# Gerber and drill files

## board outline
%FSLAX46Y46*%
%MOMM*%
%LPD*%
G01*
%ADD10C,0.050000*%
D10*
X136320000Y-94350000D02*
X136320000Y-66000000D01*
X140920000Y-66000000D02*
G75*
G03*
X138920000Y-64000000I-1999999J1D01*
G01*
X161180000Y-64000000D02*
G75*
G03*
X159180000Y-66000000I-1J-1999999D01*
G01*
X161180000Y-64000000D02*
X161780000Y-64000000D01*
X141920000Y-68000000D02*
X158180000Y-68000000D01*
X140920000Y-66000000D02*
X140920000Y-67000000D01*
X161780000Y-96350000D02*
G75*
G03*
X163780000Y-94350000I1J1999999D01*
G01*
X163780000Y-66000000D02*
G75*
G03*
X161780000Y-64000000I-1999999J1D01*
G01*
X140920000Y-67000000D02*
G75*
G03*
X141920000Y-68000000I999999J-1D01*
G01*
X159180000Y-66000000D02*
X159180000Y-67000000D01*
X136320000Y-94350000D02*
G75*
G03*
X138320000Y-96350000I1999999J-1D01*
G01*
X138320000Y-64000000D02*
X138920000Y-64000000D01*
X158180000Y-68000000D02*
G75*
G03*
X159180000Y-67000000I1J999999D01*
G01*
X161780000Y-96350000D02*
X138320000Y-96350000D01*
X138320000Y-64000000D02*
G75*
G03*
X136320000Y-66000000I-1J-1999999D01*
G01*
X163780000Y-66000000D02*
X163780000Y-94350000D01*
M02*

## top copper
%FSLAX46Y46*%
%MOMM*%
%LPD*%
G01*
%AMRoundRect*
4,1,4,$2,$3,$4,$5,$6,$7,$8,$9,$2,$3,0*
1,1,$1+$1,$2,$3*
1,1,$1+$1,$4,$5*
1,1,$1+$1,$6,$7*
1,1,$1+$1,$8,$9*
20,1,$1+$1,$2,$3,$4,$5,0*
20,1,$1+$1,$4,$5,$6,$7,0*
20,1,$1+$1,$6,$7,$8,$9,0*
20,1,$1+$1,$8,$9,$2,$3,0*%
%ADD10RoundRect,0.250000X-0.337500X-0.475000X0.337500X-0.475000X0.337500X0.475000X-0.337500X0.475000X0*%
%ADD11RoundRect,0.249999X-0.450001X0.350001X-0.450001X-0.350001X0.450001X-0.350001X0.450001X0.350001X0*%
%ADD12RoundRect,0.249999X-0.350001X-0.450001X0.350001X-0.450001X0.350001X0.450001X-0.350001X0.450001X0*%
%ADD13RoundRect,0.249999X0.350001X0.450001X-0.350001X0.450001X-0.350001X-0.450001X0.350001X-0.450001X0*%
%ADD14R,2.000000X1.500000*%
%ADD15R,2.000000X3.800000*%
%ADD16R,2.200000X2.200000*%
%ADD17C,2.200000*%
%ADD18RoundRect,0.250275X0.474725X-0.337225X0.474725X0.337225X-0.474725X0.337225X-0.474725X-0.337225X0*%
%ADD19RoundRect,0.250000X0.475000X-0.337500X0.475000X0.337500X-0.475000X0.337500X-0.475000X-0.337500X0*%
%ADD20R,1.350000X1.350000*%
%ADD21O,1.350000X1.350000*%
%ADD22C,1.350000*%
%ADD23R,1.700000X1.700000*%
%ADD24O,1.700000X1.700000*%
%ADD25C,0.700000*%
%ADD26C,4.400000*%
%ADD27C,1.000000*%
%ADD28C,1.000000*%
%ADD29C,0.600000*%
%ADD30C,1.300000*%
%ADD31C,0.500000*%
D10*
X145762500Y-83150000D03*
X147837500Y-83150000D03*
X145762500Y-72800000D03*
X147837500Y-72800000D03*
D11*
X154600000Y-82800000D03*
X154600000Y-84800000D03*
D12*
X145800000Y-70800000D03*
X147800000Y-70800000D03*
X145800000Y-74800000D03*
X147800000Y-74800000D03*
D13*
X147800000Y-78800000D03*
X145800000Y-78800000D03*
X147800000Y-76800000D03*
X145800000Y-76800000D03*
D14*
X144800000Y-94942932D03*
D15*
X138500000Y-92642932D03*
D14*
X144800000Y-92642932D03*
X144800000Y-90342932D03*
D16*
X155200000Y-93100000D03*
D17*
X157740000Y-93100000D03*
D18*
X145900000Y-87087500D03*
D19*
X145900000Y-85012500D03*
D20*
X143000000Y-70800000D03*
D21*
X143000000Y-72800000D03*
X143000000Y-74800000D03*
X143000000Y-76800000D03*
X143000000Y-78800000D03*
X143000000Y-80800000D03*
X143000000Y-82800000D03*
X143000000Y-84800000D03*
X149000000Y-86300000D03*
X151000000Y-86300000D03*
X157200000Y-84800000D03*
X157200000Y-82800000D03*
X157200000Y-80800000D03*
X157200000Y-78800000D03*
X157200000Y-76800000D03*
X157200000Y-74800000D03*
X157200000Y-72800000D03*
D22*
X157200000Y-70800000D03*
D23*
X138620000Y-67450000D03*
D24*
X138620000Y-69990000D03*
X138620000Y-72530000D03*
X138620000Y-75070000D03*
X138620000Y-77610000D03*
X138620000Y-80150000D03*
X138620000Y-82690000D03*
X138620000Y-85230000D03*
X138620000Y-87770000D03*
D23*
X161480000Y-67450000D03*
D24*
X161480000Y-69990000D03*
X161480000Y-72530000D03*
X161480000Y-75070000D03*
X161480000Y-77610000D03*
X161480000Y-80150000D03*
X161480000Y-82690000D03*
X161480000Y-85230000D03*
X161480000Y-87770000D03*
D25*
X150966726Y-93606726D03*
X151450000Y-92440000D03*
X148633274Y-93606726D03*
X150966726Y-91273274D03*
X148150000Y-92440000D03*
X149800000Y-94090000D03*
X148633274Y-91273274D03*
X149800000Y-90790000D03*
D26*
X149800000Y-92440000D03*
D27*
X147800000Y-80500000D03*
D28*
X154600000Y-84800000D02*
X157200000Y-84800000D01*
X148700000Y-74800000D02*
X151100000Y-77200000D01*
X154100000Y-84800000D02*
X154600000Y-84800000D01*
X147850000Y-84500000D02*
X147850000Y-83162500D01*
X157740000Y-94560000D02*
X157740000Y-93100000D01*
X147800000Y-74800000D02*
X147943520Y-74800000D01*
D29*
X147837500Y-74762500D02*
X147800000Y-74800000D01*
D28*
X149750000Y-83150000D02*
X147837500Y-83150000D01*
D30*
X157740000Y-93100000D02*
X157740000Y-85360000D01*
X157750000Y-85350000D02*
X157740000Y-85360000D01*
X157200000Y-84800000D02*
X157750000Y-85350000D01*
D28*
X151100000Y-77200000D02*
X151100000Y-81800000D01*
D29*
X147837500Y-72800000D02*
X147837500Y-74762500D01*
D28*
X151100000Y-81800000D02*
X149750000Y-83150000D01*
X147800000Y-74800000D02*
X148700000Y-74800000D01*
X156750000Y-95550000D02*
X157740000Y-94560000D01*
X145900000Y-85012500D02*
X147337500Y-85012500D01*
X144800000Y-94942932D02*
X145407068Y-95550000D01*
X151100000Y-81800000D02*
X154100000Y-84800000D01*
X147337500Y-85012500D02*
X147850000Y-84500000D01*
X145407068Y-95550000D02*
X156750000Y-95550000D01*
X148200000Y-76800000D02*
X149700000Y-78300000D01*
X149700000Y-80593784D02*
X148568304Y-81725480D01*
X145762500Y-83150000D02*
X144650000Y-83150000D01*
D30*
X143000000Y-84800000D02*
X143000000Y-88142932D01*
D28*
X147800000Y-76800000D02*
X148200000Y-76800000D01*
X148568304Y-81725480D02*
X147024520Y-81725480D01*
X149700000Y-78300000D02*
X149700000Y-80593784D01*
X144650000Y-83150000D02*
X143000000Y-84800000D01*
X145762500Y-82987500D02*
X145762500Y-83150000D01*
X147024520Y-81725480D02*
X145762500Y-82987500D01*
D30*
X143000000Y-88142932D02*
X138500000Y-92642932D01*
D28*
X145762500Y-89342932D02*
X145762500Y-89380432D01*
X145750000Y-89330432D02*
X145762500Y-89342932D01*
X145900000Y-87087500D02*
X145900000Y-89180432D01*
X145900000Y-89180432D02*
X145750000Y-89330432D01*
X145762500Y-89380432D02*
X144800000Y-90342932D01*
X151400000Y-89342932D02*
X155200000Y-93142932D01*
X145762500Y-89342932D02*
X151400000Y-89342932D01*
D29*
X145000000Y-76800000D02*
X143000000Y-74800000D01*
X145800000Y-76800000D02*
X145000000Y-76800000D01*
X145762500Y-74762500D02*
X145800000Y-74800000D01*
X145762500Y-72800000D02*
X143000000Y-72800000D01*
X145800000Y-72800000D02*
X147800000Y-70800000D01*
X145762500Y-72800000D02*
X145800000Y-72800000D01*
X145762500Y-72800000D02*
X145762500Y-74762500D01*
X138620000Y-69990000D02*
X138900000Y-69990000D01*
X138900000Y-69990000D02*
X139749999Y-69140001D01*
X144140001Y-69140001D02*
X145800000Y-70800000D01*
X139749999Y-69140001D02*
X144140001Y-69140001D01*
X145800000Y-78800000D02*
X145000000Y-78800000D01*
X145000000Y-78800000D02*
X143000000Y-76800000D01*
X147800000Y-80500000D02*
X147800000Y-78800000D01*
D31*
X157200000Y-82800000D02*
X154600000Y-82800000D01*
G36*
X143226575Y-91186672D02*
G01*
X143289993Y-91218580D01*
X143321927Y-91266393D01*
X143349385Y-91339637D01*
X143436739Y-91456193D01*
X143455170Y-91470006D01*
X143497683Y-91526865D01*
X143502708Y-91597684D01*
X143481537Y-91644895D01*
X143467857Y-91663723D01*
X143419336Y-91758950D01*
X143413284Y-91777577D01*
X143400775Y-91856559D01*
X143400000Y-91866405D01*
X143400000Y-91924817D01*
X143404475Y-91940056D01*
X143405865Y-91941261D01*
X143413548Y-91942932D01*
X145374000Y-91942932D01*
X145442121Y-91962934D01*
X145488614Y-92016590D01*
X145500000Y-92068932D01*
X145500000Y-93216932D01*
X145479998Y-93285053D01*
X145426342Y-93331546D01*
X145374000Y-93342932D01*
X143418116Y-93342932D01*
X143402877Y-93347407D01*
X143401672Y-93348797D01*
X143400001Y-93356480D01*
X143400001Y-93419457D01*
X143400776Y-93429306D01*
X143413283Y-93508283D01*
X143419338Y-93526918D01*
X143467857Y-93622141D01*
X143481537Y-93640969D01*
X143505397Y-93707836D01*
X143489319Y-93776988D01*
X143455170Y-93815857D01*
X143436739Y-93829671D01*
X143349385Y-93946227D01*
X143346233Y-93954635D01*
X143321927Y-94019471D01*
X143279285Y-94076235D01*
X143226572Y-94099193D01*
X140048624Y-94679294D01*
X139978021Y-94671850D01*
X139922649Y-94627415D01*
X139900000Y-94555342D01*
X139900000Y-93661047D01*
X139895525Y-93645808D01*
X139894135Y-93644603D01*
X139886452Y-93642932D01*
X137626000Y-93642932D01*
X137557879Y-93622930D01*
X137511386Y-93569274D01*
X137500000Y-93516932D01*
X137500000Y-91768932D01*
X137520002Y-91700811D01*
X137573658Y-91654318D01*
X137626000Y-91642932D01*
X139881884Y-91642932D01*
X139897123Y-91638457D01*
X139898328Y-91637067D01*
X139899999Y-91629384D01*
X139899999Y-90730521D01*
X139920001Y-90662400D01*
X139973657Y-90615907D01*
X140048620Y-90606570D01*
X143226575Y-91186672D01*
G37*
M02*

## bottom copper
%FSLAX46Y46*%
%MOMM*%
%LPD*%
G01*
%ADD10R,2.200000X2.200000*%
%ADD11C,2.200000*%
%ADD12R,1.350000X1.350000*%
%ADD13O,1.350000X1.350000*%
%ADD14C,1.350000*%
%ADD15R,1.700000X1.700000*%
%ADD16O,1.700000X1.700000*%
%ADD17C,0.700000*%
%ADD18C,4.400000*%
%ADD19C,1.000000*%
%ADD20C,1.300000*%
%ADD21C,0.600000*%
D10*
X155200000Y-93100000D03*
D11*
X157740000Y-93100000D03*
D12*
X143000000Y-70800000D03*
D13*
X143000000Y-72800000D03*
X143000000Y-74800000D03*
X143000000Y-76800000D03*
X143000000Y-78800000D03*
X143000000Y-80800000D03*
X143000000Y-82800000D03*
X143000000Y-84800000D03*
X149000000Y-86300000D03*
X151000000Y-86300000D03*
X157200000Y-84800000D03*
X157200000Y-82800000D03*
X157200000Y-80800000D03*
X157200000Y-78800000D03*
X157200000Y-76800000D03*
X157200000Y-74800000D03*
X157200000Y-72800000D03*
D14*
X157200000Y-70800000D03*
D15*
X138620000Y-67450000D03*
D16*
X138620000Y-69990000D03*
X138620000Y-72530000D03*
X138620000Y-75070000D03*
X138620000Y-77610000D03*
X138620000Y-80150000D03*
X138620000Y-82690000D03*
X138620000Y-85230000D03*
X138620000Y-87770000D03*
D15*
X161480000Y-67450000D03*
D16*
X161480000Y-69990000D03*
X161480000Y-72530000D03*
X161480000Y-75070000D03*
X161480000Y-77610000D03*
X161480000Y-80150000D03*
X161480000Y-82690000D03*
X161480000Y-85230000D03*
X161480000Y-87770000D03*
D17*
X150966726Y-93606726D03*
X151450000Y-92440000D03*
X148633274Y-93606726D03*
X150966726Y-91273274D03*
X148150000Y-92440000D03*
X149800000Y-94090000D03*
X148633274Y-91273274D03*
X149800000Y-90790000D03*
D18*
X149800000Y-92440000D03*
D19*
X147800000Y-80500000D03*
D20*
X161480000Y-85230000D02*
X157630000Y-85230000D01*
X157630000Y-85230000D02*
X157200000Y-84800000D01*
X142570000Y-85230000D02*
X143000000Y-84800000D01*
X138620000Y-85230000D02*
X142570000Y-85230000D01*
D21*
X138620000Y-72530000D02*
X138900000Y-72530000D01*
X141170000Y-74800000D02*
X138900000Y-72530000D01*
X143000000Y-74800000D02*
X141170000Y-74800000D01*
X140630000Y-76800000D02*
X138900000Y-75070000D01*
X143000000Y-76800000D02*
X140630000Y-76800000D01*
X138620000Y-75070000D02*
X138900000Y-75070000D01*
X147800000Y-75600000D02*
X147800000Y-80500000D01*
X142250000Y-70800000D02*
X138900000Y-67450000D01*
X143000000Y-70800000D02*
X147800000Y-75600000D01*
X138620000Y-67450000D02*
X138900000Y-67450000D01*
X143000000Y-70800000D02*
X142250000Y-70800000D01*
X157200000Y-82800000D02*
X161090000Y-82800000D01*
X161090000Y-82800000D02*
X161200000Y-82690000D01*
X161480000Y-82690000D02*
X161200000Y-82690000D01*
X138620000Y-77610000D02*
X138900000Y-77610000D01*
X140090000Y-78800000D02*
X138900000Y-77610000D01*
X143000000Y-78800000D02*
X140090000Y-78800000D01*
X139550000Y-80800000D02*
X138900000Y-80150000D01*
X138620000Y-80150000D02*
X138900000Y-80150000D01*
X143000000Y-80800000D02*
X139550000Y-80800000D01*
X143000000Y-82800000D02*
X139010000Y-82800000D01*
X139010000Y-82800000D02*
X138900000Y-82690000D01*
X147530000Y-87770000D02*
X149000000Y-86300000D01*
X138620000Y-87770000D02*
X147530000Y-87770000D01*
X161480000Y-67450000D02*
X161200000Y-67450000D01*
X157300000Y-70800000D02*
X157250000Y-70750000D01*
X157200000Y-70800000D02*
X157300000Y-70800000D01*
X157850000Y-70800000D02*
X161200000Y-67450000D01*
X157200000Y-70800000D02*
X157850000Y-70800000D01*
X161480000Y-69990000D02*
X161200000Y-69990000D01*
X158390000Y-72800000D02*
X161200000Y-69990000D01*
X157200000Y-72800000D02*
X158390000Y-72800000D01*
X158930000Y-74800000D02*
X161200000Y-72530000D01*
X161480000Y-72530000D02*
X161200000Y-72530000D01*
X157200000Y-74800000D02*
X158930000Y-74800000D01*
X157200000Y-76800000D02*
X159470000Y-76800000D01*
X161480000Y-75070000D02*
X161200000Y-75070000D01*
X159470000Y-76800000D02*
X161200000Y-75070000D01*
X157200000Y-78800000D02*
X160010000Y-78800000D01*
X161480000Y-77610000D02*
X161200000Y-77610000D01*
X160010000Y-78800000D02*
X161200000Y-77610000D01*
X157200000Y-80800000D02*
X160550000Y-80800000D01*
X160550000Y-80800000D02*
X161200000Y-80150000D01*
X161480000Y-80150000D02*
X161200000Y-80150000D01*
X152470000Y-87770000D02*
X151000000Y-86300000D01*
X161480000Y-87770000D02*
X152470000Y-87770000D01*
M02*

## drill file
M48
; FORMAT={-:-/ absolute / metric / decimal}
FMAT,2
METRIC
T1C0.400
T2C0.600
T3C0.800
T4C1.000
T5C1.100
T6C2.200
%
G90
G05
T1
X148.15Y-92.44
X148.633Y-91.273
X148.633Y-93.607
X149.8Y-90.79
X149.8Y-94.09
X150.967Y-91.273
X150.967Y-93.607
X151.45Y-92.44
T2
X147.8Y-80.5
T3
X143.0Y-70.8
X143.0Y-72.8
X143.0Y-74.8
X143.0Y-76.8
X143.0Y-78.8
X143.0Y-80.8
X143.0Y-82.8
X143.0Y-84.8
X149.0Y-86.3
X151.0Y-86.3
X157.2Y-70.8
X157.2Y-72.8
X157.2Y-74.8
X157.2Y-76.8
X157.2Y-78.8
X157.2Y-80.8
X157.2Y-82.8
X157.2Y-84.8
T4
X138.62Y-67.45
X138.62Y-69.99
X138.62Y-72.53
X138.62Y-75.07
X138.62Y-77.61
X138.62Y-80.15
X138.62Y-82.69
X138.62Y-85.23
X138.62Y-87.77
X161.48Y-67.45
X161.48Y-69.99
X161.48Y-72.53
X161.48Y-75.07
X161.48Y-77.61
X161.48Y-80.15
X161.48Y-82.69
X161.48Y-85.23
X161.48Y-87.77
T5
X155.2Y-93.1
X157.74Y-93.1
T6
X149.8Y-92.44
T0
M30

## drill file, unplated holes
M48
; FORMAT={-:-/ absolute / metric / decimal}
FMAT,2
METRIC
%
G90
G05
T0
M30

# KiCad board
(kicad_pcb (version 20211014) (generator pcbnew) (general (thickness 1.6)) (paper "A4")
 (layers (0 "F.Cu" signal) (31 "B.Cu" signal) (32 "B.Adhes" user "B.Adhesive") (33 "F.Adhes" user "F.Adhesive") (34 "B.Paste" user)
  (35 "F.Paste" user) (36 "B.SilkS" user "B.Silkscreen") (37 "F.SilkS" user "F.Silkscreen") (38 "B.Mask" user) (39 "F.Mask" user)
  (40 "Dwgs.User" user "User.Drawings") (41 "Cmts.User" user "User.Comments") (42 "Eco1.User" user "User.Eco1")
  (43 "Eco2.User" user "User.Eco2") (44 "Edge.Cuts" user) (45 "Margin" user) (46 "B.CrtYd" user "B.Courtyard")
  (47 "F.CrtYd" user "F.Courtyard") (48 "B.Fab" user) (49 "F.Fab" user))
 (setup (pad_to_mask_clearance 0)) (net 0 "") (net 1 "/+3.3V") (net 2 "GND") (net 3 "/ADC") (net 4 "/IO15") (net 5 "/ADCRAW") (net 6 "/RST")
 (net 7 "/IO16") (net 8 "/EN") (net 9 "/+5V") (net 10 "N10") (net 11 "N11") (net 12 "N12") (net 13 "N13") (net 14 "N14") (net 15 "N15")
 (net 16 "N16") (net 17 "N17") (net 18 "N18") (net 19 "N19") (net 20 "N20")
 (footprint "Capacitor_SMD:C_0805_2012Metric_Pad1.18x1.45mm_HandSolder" (layer "F.Cu") (at 146.8 83.15)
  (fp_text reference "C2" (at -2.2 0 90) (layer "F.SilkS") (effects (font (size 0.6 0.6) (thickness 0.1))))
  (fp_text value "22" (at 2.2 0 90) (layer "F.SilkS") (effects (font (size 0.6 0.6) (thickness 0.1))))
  (pad "1" smd roundrect locked (at -1.0375 0) (size 1.175 1.45) (layers "F.Cu" "F.Paste" "F.Mask") (roundrect_rratio 0.2127659574)
   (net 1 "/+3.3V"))
  (pad "2" smd roundrect locked (at 1.0375 0) (size 1.175 1.45) (layers "F.Cu" "F.Paste" "F.Mask") (roundrect_rratio 0.2127659574)
   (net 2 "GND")))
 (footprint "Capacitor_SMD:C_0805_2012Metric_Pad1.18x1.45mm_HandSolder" (layer "F.Cu") (at 146.8 72.8)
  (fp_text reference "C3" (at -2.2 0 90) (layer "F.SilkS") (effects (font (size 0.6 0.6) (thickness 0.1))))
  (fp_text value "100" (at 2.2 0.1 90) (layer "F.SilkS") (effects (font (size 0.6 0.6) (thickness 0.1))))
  (pad "1" smd roundrect locked (at -1.0375 0) (size 1.175 1.45) (layers "F.Cu" "F.Paste" "F.Mask") (roundrect_rratio 0.2127659574)
   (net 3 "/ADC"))
  (pad "2" smd roundrect locked (at 1.0375 0) (size 1.175 1.45) (layers "F.Cu" "F.Paste" "F.Mask") (roundrect_rratio 0.2127659574)
   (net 2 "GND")))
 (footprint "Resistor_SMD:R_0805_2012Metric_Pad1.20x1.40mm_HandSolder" (layer "F.Cu") (at 154.6 83.8 -90)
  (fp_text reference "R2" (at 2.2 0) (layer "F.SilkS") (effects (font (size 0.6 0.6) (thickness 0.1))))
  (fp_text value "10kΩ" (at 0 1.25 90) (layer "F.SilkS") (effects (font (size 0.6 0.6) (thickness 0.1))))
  (pad "1" smd roundrect locked (at -1 0 270) (size 1.2 1.4) (layers "F.Cu" "F.Paste" "F.Mask") (roundrect_rratio 0.2083325) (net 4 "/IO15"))
  (pad "2" smd roundrect locked (at 1 0 270) (size 1.2 1.4) (layers "F.Cu" "F.Paste" "F.Mask") (roundrect_rratio 0.2083325) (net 2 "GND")))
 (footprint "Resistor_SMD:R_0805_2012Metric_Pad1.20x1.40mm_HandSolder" (layer "F.Cu") (at 146.8 70.8)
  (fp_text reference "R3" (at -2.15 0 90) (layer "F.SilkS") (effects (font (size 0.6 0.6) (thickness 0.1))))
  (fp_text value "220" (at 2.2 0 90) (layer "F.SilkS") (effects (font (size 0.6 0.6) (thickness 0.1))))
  (pad "1" smd roundrect locked (at -1 0) (size 1.2 1.4) (layers "F.Cu" "F.Paste" "F.Mask") (roundrect_rratio 0.2083325) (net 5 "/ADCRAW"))
  (pad "2" smd roundrect locked (at 1 0) (size 1.2 1.4) (layers "F.Cu" "F.Paste" "F.Mask") (roundrect_rratio 0.2083325) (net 3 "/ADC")))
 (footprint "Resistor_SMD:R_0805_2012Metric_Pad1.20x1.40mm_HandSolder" (layer "F.Cu") (at 146.8 74.8)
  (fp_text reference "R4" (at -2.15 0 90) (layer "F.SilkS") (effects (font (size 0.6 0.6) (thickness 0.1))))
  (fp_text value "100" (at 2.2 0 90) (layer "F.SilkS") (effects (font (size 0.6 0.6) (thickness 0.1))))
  (pad "1" smd roundrect locked (at -1 0) (size 1.2 1.4) (layers "F.Cu" "F.Paste" "F.Mask") (roundrect_rratio 0.2083325) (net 3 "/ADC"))
  (pad "2" smd roundrect locked (at 1 0) (size 1.2 1.4) (layers "F.Cu" "F.Paste" "F.Mask") (roundrect_rratio 0.2083325) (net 2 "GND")))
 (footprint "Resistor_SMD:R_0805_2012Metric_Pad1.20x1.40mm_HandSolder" (layer "F.Cu") (at 146.8 78.8 180)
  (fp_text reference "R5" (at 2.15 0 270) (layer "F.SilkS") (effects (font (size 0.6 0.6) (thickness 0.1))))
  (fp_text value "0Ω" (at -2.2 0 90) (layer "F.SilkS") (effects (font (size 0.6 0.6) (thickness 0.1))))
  (pad "1" smd roundrect locked (at -1 0 180) (size 1.2 1.4) (layers "F.Cu" "F.Paste" "F.Mask") (roundrect_rratio 0.2083325) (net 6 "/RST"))
  (pad "2" smd roundrect locked (at 1 0 180) (size 1.2 1.4) (layers "F.Cu" "F.Paste" "F.Mask") (roundrect_rratio 0.2083325) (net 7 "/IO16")))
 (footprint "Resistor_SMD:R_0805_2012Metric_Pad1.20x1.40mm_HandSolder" (layer "F.Cu") (at 146.8 76.8 180)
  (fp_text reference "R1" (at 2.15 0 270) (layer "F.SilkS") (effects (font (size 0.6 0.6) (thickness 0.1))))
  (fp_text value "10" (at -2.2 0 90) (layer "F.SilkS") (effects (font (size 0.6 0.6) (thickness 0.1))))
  (pad "1" smd roundrect locked (at -1 0 180) (size 1.2 1.4) (layers "F.Cu" "F.Paste" "F.Mask") (roundrect_rratio 0.2083325)
   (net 1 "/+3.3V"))
  (pad "2" smd roundrect locked (at 1 0 180) (size 1.2 1.4) (layers "F.Cu" "F.Paste" "F.Mask") (roundrect_rratio 0.2083325) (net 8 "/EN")))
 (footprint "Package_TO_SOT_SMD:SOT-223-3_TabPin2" (layer "F.Cu") (at 141.65 92.642932 180)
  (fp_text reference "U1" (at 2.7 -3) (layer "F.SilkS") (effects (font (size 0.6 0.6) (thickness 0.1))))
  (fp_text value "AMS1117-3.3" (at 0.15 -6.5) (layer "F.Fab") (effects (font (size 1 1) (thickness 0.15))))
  (pad "1" smd rect locked (at -3.15 -2.3 180) (size 2 1.5) (layers "F.Cu" "F.Paste" "F.Mask") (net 2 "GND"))
  (pad "2" smd rect locked (at 3.15 0 180) (size 2 3.8) (layers "F.Cu" "F.Paste" "F.Mask") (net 1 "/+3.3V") (zone_connect 1)
   (thermal_width 3.3) (thermal_gap 0.4))
  (pad "2" smd rect locked (at -3.15 0 180) (size 2 1.5) (layers "F.Cu" "F.Paste" "F.Mask") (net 1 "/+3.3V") (zone_connect 1)
   (thermal_width 1.4) (thermal_gap 0.4))
  (pad "3" smd rect locked (at -3.15 2.3 180) (size 2 1.5) (layers "F.Cu" "F.Paste" "F.Mask") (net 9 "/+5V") (zone_connect 1)
   (thermal_width 1) (thermal_gap 0.5)))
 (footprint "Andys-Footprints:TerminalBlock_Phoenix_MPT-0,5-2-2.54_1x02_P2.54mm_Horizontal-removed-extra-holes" (layer "F.Cu")
  (at 155.2 93.1)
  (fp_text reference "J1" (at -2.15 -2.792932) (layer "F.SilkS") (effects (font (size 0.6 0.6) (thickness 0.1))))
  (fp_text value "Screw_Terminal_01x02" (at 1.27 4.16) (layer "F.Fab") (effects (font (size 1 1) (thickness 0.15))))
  (pad "1" thru_hole rect locked (at 0 0) (size 2.2 2.2) (drill 1.1) (layers *.Cu *.Mask) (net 9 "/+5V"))
  (pad "2" thru_hole circle locked (at 2.54 0) (size 2.2 2.2) (drill 1.1) (layers *.Cu *.Mask) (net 2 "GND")))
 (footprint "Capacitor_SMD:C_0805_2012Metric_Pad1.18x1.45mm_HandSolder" (layer "F.Cu") (at 145.9 86.05 90)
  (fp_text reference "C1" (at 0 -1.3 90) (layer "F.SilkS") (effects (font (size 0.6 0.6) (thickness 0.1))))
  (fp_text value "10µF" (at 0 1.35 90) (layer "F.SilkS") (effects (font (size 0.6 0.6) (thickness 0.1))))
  (pad "1" smd roundrect locked (at -1.0375 0 90) (size 1.175 1.45) (layers "F.Cu" "F.Paste" "F.Mask") (roundrect_rratio 0.213)
   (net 9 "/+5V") (zone_connect 1) (thermal_width 1) (thermal_gap 0.5))
  (pad "2" smd roundrect locked (at 1.0375 0 90) (size 1.175 1.45) (layers "F.Cu" "F.Paste" "F.Mask") (roundrect_rratio 0.2127659574)
   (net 2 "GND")))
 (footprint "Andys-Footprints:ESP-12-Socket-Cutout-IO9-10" (layer "F.Cu") (at 143 70.8)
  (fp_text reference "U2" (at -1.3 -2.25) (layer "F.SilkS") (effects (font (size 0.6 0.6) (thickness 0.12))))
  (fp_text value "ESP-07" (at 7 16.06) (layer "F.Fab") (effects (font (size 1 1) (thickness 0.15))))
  (pad "1" thru_hole rect (at 0 0) (size 1.35 1.35) (drill 0.8) (layers *.Cu *.Mask) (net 6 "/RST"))
  (pad "2" thru_hole oval (at 0 2) (size 1.35 1.35) (drill 0.8) (layers *.Cu *.Mask) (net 3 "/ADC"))
  (pad "3" thru_hole oval (at 0 4) (size 1.35 1.35) (drill 0.8) (layers *.Cu *.Mask) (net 8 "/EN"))
  (pad "4" thru_hole oval (at 0 6) (size 1.35 1.35) (drill 0.8) (layers *.Cu *.Mask) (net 7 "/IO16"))
  (pad "5" thru_hole oval (at 0 8) (size 1.35 1.35) (drill 0.8) (layers *.Cu *.Mask) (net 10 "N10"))
  (pad "6" thru_hole oval (at 0 10) (size 1.35 1.35) (drill 0.8) (layers *.Cu *.Mask) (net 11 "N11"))
  (pad "7" thru_hole oval (at 0 12) (size 1.35 1.35) (drill 0.8) (layers *.Cu *.Mask) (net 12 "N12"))
  (pad "8" thru_hole oval (at 0 14) (size 1.35 1.35) (drill 0.8) (layers *.Cu *.Mask) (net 1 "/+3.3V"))
  (pad "11" thru_hole oval (at 6 15.5 270) (size 1.35 1.35) (drill 0.8) (layers *.Cu *.Mask) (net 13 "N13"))
  (pad "12" thru_hole oval (at 8 15.5 270) (size 1.35 1.35) (drill 0.8) (layers *.Cu *.Mask) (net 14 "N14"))
  (pad "15" thru_hole oval (at 14.2 14) (size 1.35 1.35) (drill 0.8) (layers *.Cu *.Mask) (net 2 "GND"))
  (pad "16" thru_hole oval (at 14.2 12) (size 1.35 1.35) (drill 0.8) (layers *.Cu *.Mask) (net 4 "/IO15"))
  (pad "17" thru_hole oval (at 14.2 10) (size 1.35 1.35) (drill 0.8) (layers *.Cu *.Mask) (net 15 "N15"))
  (pad "18" thru_hole oval (at 14.2 8) (size 1.35 1.35) (drill 0.8) (layers *.Cu *.Mask) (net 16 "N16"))
  (pad "19" thru_hole oval (at 14.2 6) (size 1.35 1.35) (drill 0.8) (layers *.Cu *.Mask) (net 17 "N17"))
  (pad "20" thru_hole oval (at 14.2 4) (size 1.35 1.35) (drill 0.8) (layers *.Cu *.Mask) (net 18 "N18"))
  (pad "21" thru_hole oval (at 14.2 2) (size 1.35 1.35) (drill 0.8) (layers *.Cu *.Mask) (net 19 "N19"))
  (pad "22" thru_hole circle (at 14.2 0) (size 1.35 1.35) (drill 0.8) (layers *.Cu *.Mask) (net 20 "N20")))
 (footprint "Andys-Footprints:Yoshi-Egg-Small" (layer "F.Cu") (at 161.45 92.35)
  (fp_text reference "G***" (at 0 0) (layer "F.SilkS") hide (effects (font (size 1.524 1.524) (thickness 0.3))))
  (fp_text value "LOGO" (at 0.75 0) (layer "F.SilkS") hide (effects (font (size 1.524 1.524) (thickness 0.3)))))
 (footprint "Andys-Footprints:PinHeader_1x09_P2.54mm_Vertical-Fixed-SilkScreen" (layer "F.Cu") (at 138.62 67.45)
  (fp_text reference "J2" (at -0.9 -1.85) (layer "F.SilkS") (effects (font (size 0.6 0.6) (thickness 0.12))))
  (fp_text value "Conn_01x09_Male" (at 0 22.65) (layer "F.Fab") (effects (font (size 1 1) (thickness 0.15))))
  (pad "1" thru_hole rect (at 0 0) (size 1.7 1.7) (drill 1) (layers *.Cu *.Mask) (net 6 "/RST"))
  (pad "2" thru_hole oval (at 0 2.54) (size 1.7 1.7) (drill 1) (layers *.Cu *.Mask) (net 5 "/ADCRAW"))
  (pad "3" thru_hole oval (at 0 5.08) (size 1.7 1.7) (drill 1) (layers *.Cu *.Mask) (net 8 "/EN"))
  (pad "4" thru_hole oval (at 0 7.62) (size 1.7 1.7) (drill 1) (layers *.Cu *.Mask) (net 7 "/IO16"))
  (pad "5" thru_hole oval (at 0 10.16) (size 1.7 1.7) (drill 1) (layers *.Cu *.Mask) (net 10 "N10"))
  (pad "6" thru_hole oval (at 0 12.7) (size 1.7 1.7) (drill 1) (layers *.Cu *.Mask) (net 11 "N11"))
  (pad "7" thru_hole oval (at 0 15.24) (size 1.7 1.7) (drill 1) (layers *.Cu *.Mask) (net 12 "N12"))
  (pad "8" thru_hole oval (at 0 17.78) (size 1.7 1.7) (drill 1) (layers *.Cu *.Mask) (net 1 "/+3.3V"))
  (pad "9" thru_hole oval (at 0 20.32) (size 1.7 1.7) (drill 1) (layers *.Cu *.Mask) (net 13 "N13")))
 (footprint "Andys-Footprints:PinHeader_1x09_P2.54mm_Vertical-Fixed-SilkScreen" (layer "F.Cu") (at 161.48 67.45)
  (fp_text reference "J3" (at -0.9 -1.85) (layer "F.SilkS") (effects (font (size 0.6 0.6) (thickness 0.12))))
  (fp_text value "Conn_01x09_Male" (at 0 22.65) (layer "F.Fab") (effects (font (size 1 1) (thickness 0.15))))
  (pad "1" thru_hole rect (at 0 0) (size 1.7 1.7) (drill 1) (layers *.Cu *.Mask) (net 20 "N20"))
  (pad "2" thru_hole oval (at 0 2.54) (size 1.7 1.7) (drill 1) (layers *.Cu *.Mask) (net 19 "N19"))
  (pad "3" thru_hole oval (at 0 5.08) (size 1.7 1.7) (drill 1) (layers *.Cu *.Mask) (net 18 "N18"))
  (pad "4" thru_hole oval (at 0 7.62) (size 1.7 1.7) (drill 1) (layers *.Cu *.Mask) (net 17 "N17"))
  (pad "5" thru_hole oval (at 0 10.16) (size 1.7 1.7) (drill 1) (layers *.Cu *.Mask) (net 16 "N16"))
  (pad "6" thru_hole oval (at 0 12.7) (size 1.7 1.7) (drill 1) (layers *.Cu *.Mask) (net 15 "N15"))
  (pad "7" thru_hole oval (at 0 15.24) (size 1.7 1.7) (drill 1) (layers *.Cu *.Mask) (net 4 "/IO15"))
  (pad "8" thru_hole oval (at 0 17.78) (size 1.7 1.7) (drill 1) (layers *.Cu *.Mask) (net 2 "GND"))
  (pad "9" thru_hole oval (at 0 20.32) (size 1.7 1.7) (drill 1) (layers *.Cu *.Mask) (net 14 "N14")))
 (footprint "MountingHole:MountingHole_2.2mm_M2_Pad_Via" (layer "F.Cu") (at 149.8 92.44)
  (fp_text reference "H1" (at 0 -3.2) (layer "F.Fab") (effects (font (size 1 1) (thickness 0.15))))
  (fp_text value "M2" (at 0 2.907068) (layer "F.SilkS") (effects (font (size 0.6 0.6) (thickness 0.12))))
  (pad "1" thru_hole circle locked (at 1.166726 1.166726) (size 0.7 0.7) (drill 0.4) (layers *.Cu *.Mask))
  (pad "1" thru_hole circle locked (at 1.65 0) (size 0.7 0.7) (drill 0.4) (layers *.Cu *.Mask))
  (pad "1" thru_hole circle locked (at -1.166726 1.166726) (size 0.7 0.7) (drill 0.4) (layers *.Cu *.Mask))
  (pad "1" thru_hole circle locked (at 1.166726 -1.166726) (size 0.7 0.7) (drill 0.4) (layers *.Cu *.Mask))
  (pad "1" thru_hole circle locked (at -1.65 0) (size 0.7 0.7) (drill 0.4) (layers *.Cu *.Mask))
  (pad "1" thru_hole circle locked (at 0 1.65) (size 0.7 0.7) (drill 0.4) (layers *.Cu *.Mask))
  (pad "1" thru_hole circle locked (at -1.166726 -1.166726) (size 0.7 0.7) (drill 0.4) (layers *.Cu *.Mask))
  (pad "1" thru_hole circle locked (at 0 -1.65) (size 0.7 0.7) (drill 0.4) (layers *.Cu *.Mask))
  (pad "1" thru_hole circle locked (at 0 0) (size 4.4 4.4) (drill 2.2) (layers *.Cu *.Mask)))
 (gr_line (start 136.32 94.35) (end 136.32 66) (layer "Edge.Cuts") (width 0.05))
 (gr_arc (start 138.92 64) (mid 140.334214 64.585786) (end 140.92 66) (layer "Edge.Cuts") (width 0.05))
 (gr_arc (start 159.18 66) (mid 159.765786 64.585786) (end 161.18 64) (layer "Edge.Cuts") (width 0.05))
 (gr_line (start 161.18 64) (end 161.78 64) (layer "Edge.Cuts") (width 0.05))
 (gr_line (start 141.92 68) (end 158.18 68) (layer "Edge.Cuts") (width 0.05))
 (gr_line (start 140.92 66) (end 140.92 67) (layer "Edge.Cuts") (width 0.05))
 (gr_arc (start 163.78 94.35) (mid 163.194214 95.764214) (end 161.78 96.35) (layer "Edge.Cuts") (width 0.05))
 (gr_arc (start 161.78 64) (mid 163.194214 64.585786) (end 163.78 66) (layer "Edge.Cuts") (width 0.05))
 (gr_arc (start 141.92 68) (mid 141.212893 67.707107) (end 140.92 67) (layer "Edge.Cuts") (width 0.05))
 (gr_line (start 159.18 66) (end 159.18 67) (layer "Edge.Cuts") (width 0.05))
 (gr_arc (start 138.32 96.35) (mid 136.905786 95.764214) (end 136.32 94.35) (layer "Edge.Cuts") (width 0.05))
 (gr_line (start 138.32 64) (end 138.92 64) (layer "Edge.Cuts") (width 0.05))
 (gr_arc (start 159.18 67) (mid 158.887107 67.707107) (end 158.18 68) (layer "Edge.Cuts") (width 0.05))
 (gr_line (start 161.78 96.35) (end 138.32 96.35) (layer "Edge.Cuts") (width 0.05))
 (gr_arc (start 136.32 66) (mid 136.905786 64.585786) (end 138.32 64) (layer "Edge.Cuts") (width 0.05))
 (gr_line (start 163.78 66) (end 163.78 94.35) (layer "Edge.Cuts") (width 0.05))
 (segment (start 154.6 84.8) (end 157.2 84.8) (width 1) (layer "F.Cu") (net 2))
 (segment (start 148.7 74.8) (end 151.1 77.2) (width 1) (layer "F.Cu") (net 2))
 (segment (start 154.1 84.8) (end 154.6 84.8) (width 1) (layer "F.Cu") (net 2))
 (segment (start 147.85 84.5) (end 147.85 83.1625) (width 1) (layer "F.Cu") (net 2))
 (segment (start 157.74 94.56) (end 157.74 93.1) (width 1) (layer "F.Cu") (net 2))
 (segment (start 147.8 74.8) (end 147.94352 74.8) (width 1) (layer "F.Cu") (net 2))
 (segment (start 147.8375 74.7625) (end 147.8 74.8) (width 0.6) (layer "F.Cu") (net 2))
 (segment (start 149.75 83.15) (end 147.8375 83.15) (width 1) (layer "F.Cu") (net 2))
 (segment (start 157.74 93.1) (end 157.74 85.36) (width 1.3) (layer "F.Cu") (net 2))
 (segment (start 157.75 85.35) (end 157.74 85.36) (width 1.3) (layer "F.Cu") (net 2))
 (segment (start 157.2 84.8) (end 157.75 85.35) (width 1.3) (layer "F.Cu") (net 2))
 (segment (start 151.1 77.2) (end 151.1 81.8) (width 1) (layer "F.Cu") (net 2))
 (segment (start 147.8375 72.8) (end 147.8375 74.7625) (width 0.6) (layer "F.Cu") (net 2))
 (segment (start 151.1 81.8) (end 149.75 83.15) (width 1) (layer "F.Cu") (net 2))
 (segment (start 147.8 74.8) (end 148.7 74.8) (width 1) (layer "F.Cu") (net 2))
 (segment (start 156.75 95.55) (end 157.74 94.56) (width 1) (layer "F.Cu") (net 2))
 (segment (start 145.9 85.0125) (end 147.3375 85.0125) (width 1) (layer "F.Cu") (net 2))
 (segment (start 144.8 94.942932) (end 145.407068 95.55) (width 1) (layer "F.Cu") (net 2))
 (segment (start 151.1 81.8) (end 154.1 84.8) (width 1) (layer "F.Cu") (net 2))
 (segment (start 147.3375 85.0125) (end 147.85 84.5) (width 1) (layer "F.Cu") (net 2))
 (segment (start 145.407068 95.55) (end 156.75 95.55) (width 1) (layer "F.Cu") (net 2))
 (segment (start 161.48 85.23) (end 157.63 85.23) (width 1.3) (layer "B.Cu") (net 2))
 (segment (start 157.63 85.23) (end 157.2 84.8) (width 1.3) (layer "B.Cu") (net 2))
 (segment (start 148.2 76.8) (end 149.7 78.3) (width 1) (layer "F.Cu") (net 1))
 (segment (start 149.7 80.593784) (end 148.568304 81.72548) (width 1) (layer "F.Cu") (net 1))
 (segment (start 145.7625 83.15) (end 144.65 83.15) (width 1) (layer "F.Cu") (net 1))
 (segment (start 143 84.8) (end 143 88.142932) (width 1.3) (layer "F.Cu") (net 1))
 (segment (start 147.8 76.8) (end 148.2 76.8) (width 1) (layer "F.Cu") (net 1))
 (segment (start 148.568304 81.72548) (end 147.02452 81.72548) (width 1) (layer "F.Cu") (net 1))
 (segment (start 149.7 78.3) (end 149.7 80.593784) (width 1) (layer "F.Cu") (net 1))
 (segment (start 144.65 83.15) (end 143 84.8) (width 1) (layer "F.Cu") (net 1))
 (segment (start 145.7625 82.9875) (end 145.7625 83.15) (width 1) (layer "F.Cu") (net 1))
 (segment (start 147.02452 81.72548) (end 145.7625 82.9875) (width 1) (layer "F.Cu") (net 1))
 (segment (start 143 88.142932) (end 138.5 92.642932) (width 1.3) (layer "F.Cu") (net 1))
 (segment (start 142.57 85.23) (end 143 84.8) (width 1.3) (layer "B.Cu") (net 1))
 (segment (start 138.62 85.23) (end 142.57 85.23) (width 1.3) (layer "B.Cu") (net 1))
 (segment (start 145.7625 89.342932) (end 145.7625 89.380432) (width 1) (layer "F.Cu") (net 9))
 (segment (start 145.75 89.330432) (end 145.7625 89.342932) (width 1) (layer "F.Cu") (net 9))
 (segment (start 145.9 87.0875) (end 145.9 89.180432) (width 1) (layer "F.Cu") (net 9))
 (segment (start 145.9 89.180432) (end 145.75 89.330432) (width 1) (layer "F.Cu") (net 9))
 (segment (start 145.7625 89.380432) (end 144.8 90.342932) (width 1) (layer "F.Cu") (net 9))
 (segment (start 151.4 89.342932) (end 155.2 93.142932) (width 1) (layer "F.Cu") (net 9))
 (segment (start 145.7625 89.342932) (end 151.4 89.342932) (width 1) (layer "F.Cu") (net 9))
 (segment (start 145 76.8) (end 143 74.8) (width 0.6) (layer "F.Cu") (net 8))
 (segment (start 145.8 76.8) (end 145 76.8) (width 0.6) (layer "F.Cu") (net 8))
 (segment (start 138.62 72.53) (end 138.9 72.53) (width 0.6) (layer "B.Cu") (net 8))
 (segment (start 141.17 74.8) (end 138.9 72.53) (width 0.6) (layer "B.Cu") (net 8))
 (segment (start 143 74.8) (end 141.17 74.8) (width 0.6) (layer "B.Cu") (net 8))
 (segment (start 145.7625 74.7625) (end 145.8 74.8) (width 0.6) (layer "F.Cu") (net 3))
 (segment (start 145.7625 72.8) (end 143 72.8) (width 0.6) (layer "F.Cu") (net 3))
 (segment (start 145.8 72.8) (end 147.8 70.8) (width 0.6) (layer "F.Cu") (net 3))
 (segment (start 145.7625 72.8) (end 145.8 72.8) (width 0.6) (layer "F.Cu") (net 3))
 (segment (start 145.7625 72.8) (end 145.7625 74.7625) (width 0.6) (layer "F.Cu") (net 3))
 (segment (start 138.62 69.99) (end 138.9 69.99) (width 0.6) (layer "F.Cu") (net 5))
 (segment (start 138.9 69.99) (end 139.749999 69.140001) (width 0.6) (layer "F.Cu") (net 5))
 (segment (start 144.140001 69.140001) (end 145.8 70.8) (width 0.6) (layer "F.Cu") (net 5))
 (segment (start 139.749999 69.140001) (end 144.140001 69.140001) (width 0.6) (layer "F.Cu") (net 5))
 (segment (start 145.8 78.8) (end 145 78.8) (width 0.6) (layer "F.Cu") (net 7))
 (segment (start 145 78.8) (end 143 76.8) (width 0.6) (layer "F.Cu") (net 7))
 (segment (start 140.63 76.8) (end 138.9 75.07) (width 0.6) (layer "B.Cu") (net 7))
 (segment (start 143 76.8) (end 140.63 76.8) (width 0.6) (layer "B.Cu") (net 7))
 (segment (start 138.62 75.07) (end 138.9 75.07) (width 0.6) (layer "B.Cu") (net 7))
 (segment (start 147.8 80.5) (end 147.8 78.8) (width 0.6) (layer "F.Cu") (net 6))
 (via (at 147.8 80.5) (size 1) (drill 0.6) (layers "F.Cu" "B.Cu") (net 6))
 (segment (start 147.8 75.6) (end 147.8 80.5) (width 0.6) (layer "B.Cu") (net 6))
 (segment (start 142.25 70.8) (end 138.9 67.45) (width 0.6) (layer "B.Cu") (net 6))
 (segment (start 143 70.8) (end 147.8 75.6) (width 0.6) (layer "B.Cu") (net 6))
 (segment (start 138.62 67.45) (end 138.9 67.45) (width 0.6) (layer "B.Cu") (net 6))
 (segment (start 143 70.8) (end 142.25 70.8) (width 0.6) (layer "B.Cu") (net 6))
 (segment (start 157.2 82.8) (end 154.6 82.8) (width 0.5) (layer "F.Cu") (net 4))
 (segment (start 157.2 82.8) (end 161.09 82.8) (width 0.6) (layer "B.Cu") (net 4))
 (segment (start 161.09 82.8) (end 161.2 82.69) (width 0.6) (layer "B.Cu") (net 4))
 (segment (start 161.48 82.69) (end 161.2 82.69) (width 0.6) (layer "B.Cu") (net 4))
 (segment (start 138.62 77.61) (end 138.9 77.61) (width 0.6) (layer "B.Cu") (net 10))
 (segment (start 140.09 78.8) (end 138.9 77.61) (width 0.6) (layer "B.Cu") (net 10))
 (segment (start 143 78.8) (end 140.09 78.8) (width 0.6) (layer "B.Cu") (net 10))
 (segment (start 139.55 80.8) (end 138.9 80.15) (width 0.6) (layer "B.Cu") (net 11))
 (segment (start 138.62 80.15) (end 138.9 80.15) (width 0.6) (layer "B.Cu") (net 11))
 (segment (start 143 80.8) (end 139.55 80.8) (width 0.6) (layer "B.Cu") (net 11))
 (segment (start 143 82.8) (end 139.01 82.8) (width 0.6) (layer "B.Cu") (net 12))
 (segment (start 139.01 82.8) (end 138.9 82.69) (width 0.6) (layer "B.Cu") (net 12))
 (segment (start 147.53 87.77) (end 149 86.3) (width 0.6) (layer "B.Cu") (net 13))
 (segment (start 138.62 87.77) (end 147.53 87.77) (width 0.6) (layer "B.Cu") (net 13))
 (segment (start 161.48 67.45) (end 161.2 67.45) (width 0.6) (layer "B.Cu") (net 20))
 (segment (start 157.3 70.8) (end 157.25 70.75) (width 0.6) (layer "B.Cu") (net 20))
 (segment (start 157.2 70.8) (end 157.3 70.8) (width 0.6) (layer "B.Cu") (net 20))
 (segment (start 157.85 70.8) (end 161.2 67.45) (width 0.6) (layer "B.Cu") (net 20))
 (segment (start 157.2 70.8) (end 157.85 70.8) (width 0.6) (layer "B.Cu") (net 20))
 (segment (start 161.48 69.99) (end 161.2 69.99) (width 0.6) (layer "B.Cu") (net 19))
 (segment (start 158.39 72.8) (end 161.2 69.99) (width 0.6) (layer "B.Cu") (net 19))
 (segment (start 157.2 72.8) (end 158.39 72.8) (width 0.6) (layer "B.Cu") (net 19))
 (segment (start 158.93 74.8) (end 161.2 72.53) (width 0.6) (layer "B.Cu") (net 18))
 (segment (start 161.48 72.53) (end 161.2 72.53) (width 0.6) (layer "B.Cu") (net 18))
 (segment (start 157.2 74.8) (end 158.93 74.8) (width 0.6) (layer "B.Cu") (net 18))
 (segment (start 157.2 76.8) (end 159.47 76.8) (width 0.6) (layer "B.Cu") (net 17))
 (segment (start 161.48 75.07) (end 161.2 75.07) (width 0.6) (layer "B.Cu") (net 17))
 (segment (start 159.47 76.8) (end 161.2 75.07) (width 0.6) (layer "B.Cu") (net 17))
 (segment (start 157.2 78.8) (end 160.01 78.8) (width 0.6) (layer "B.Cu") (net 16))
 (segment (start 161.48 77.61) (end 161.2 77.61) (width 0.6) (layer "B.Cu") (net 16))
 (segment (start 160.01 78.8) (end 161.2 77.61) (width 0.6) (layer "B.Cu") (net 16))
 (segment (start 157.2 80.8) (end 160.55 80.8) (width 0.6) (layer "B.Cu") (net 15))
 (segment (start 160.55 80.8) (end 161.2 80.15) (width 0.6) (layer "B.Cu") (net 15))
 (segment (start 161.48 80.15) (end 161.2 80.15) (width 0.6) (layer "B.Cu") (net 15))
 (segment (start 152.47 87.77) (end 151 86.3) (width 0.6) (layer "B.Cu") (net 14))
 (segment (start 161.48 87.77) (end 152.47 87.77) (width 0.6) (layer "B.Cu") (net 14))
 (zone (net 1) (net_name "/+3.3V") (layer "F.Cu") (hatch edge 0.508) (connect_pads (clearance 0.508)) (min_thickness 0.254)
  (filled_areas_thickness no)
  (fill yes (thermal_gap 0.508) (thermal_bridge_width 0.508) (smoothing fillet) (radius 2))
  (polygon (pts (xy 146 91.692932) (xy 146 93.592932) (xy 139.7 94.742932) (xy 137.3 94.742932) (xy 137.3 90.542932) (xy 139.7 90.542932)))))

